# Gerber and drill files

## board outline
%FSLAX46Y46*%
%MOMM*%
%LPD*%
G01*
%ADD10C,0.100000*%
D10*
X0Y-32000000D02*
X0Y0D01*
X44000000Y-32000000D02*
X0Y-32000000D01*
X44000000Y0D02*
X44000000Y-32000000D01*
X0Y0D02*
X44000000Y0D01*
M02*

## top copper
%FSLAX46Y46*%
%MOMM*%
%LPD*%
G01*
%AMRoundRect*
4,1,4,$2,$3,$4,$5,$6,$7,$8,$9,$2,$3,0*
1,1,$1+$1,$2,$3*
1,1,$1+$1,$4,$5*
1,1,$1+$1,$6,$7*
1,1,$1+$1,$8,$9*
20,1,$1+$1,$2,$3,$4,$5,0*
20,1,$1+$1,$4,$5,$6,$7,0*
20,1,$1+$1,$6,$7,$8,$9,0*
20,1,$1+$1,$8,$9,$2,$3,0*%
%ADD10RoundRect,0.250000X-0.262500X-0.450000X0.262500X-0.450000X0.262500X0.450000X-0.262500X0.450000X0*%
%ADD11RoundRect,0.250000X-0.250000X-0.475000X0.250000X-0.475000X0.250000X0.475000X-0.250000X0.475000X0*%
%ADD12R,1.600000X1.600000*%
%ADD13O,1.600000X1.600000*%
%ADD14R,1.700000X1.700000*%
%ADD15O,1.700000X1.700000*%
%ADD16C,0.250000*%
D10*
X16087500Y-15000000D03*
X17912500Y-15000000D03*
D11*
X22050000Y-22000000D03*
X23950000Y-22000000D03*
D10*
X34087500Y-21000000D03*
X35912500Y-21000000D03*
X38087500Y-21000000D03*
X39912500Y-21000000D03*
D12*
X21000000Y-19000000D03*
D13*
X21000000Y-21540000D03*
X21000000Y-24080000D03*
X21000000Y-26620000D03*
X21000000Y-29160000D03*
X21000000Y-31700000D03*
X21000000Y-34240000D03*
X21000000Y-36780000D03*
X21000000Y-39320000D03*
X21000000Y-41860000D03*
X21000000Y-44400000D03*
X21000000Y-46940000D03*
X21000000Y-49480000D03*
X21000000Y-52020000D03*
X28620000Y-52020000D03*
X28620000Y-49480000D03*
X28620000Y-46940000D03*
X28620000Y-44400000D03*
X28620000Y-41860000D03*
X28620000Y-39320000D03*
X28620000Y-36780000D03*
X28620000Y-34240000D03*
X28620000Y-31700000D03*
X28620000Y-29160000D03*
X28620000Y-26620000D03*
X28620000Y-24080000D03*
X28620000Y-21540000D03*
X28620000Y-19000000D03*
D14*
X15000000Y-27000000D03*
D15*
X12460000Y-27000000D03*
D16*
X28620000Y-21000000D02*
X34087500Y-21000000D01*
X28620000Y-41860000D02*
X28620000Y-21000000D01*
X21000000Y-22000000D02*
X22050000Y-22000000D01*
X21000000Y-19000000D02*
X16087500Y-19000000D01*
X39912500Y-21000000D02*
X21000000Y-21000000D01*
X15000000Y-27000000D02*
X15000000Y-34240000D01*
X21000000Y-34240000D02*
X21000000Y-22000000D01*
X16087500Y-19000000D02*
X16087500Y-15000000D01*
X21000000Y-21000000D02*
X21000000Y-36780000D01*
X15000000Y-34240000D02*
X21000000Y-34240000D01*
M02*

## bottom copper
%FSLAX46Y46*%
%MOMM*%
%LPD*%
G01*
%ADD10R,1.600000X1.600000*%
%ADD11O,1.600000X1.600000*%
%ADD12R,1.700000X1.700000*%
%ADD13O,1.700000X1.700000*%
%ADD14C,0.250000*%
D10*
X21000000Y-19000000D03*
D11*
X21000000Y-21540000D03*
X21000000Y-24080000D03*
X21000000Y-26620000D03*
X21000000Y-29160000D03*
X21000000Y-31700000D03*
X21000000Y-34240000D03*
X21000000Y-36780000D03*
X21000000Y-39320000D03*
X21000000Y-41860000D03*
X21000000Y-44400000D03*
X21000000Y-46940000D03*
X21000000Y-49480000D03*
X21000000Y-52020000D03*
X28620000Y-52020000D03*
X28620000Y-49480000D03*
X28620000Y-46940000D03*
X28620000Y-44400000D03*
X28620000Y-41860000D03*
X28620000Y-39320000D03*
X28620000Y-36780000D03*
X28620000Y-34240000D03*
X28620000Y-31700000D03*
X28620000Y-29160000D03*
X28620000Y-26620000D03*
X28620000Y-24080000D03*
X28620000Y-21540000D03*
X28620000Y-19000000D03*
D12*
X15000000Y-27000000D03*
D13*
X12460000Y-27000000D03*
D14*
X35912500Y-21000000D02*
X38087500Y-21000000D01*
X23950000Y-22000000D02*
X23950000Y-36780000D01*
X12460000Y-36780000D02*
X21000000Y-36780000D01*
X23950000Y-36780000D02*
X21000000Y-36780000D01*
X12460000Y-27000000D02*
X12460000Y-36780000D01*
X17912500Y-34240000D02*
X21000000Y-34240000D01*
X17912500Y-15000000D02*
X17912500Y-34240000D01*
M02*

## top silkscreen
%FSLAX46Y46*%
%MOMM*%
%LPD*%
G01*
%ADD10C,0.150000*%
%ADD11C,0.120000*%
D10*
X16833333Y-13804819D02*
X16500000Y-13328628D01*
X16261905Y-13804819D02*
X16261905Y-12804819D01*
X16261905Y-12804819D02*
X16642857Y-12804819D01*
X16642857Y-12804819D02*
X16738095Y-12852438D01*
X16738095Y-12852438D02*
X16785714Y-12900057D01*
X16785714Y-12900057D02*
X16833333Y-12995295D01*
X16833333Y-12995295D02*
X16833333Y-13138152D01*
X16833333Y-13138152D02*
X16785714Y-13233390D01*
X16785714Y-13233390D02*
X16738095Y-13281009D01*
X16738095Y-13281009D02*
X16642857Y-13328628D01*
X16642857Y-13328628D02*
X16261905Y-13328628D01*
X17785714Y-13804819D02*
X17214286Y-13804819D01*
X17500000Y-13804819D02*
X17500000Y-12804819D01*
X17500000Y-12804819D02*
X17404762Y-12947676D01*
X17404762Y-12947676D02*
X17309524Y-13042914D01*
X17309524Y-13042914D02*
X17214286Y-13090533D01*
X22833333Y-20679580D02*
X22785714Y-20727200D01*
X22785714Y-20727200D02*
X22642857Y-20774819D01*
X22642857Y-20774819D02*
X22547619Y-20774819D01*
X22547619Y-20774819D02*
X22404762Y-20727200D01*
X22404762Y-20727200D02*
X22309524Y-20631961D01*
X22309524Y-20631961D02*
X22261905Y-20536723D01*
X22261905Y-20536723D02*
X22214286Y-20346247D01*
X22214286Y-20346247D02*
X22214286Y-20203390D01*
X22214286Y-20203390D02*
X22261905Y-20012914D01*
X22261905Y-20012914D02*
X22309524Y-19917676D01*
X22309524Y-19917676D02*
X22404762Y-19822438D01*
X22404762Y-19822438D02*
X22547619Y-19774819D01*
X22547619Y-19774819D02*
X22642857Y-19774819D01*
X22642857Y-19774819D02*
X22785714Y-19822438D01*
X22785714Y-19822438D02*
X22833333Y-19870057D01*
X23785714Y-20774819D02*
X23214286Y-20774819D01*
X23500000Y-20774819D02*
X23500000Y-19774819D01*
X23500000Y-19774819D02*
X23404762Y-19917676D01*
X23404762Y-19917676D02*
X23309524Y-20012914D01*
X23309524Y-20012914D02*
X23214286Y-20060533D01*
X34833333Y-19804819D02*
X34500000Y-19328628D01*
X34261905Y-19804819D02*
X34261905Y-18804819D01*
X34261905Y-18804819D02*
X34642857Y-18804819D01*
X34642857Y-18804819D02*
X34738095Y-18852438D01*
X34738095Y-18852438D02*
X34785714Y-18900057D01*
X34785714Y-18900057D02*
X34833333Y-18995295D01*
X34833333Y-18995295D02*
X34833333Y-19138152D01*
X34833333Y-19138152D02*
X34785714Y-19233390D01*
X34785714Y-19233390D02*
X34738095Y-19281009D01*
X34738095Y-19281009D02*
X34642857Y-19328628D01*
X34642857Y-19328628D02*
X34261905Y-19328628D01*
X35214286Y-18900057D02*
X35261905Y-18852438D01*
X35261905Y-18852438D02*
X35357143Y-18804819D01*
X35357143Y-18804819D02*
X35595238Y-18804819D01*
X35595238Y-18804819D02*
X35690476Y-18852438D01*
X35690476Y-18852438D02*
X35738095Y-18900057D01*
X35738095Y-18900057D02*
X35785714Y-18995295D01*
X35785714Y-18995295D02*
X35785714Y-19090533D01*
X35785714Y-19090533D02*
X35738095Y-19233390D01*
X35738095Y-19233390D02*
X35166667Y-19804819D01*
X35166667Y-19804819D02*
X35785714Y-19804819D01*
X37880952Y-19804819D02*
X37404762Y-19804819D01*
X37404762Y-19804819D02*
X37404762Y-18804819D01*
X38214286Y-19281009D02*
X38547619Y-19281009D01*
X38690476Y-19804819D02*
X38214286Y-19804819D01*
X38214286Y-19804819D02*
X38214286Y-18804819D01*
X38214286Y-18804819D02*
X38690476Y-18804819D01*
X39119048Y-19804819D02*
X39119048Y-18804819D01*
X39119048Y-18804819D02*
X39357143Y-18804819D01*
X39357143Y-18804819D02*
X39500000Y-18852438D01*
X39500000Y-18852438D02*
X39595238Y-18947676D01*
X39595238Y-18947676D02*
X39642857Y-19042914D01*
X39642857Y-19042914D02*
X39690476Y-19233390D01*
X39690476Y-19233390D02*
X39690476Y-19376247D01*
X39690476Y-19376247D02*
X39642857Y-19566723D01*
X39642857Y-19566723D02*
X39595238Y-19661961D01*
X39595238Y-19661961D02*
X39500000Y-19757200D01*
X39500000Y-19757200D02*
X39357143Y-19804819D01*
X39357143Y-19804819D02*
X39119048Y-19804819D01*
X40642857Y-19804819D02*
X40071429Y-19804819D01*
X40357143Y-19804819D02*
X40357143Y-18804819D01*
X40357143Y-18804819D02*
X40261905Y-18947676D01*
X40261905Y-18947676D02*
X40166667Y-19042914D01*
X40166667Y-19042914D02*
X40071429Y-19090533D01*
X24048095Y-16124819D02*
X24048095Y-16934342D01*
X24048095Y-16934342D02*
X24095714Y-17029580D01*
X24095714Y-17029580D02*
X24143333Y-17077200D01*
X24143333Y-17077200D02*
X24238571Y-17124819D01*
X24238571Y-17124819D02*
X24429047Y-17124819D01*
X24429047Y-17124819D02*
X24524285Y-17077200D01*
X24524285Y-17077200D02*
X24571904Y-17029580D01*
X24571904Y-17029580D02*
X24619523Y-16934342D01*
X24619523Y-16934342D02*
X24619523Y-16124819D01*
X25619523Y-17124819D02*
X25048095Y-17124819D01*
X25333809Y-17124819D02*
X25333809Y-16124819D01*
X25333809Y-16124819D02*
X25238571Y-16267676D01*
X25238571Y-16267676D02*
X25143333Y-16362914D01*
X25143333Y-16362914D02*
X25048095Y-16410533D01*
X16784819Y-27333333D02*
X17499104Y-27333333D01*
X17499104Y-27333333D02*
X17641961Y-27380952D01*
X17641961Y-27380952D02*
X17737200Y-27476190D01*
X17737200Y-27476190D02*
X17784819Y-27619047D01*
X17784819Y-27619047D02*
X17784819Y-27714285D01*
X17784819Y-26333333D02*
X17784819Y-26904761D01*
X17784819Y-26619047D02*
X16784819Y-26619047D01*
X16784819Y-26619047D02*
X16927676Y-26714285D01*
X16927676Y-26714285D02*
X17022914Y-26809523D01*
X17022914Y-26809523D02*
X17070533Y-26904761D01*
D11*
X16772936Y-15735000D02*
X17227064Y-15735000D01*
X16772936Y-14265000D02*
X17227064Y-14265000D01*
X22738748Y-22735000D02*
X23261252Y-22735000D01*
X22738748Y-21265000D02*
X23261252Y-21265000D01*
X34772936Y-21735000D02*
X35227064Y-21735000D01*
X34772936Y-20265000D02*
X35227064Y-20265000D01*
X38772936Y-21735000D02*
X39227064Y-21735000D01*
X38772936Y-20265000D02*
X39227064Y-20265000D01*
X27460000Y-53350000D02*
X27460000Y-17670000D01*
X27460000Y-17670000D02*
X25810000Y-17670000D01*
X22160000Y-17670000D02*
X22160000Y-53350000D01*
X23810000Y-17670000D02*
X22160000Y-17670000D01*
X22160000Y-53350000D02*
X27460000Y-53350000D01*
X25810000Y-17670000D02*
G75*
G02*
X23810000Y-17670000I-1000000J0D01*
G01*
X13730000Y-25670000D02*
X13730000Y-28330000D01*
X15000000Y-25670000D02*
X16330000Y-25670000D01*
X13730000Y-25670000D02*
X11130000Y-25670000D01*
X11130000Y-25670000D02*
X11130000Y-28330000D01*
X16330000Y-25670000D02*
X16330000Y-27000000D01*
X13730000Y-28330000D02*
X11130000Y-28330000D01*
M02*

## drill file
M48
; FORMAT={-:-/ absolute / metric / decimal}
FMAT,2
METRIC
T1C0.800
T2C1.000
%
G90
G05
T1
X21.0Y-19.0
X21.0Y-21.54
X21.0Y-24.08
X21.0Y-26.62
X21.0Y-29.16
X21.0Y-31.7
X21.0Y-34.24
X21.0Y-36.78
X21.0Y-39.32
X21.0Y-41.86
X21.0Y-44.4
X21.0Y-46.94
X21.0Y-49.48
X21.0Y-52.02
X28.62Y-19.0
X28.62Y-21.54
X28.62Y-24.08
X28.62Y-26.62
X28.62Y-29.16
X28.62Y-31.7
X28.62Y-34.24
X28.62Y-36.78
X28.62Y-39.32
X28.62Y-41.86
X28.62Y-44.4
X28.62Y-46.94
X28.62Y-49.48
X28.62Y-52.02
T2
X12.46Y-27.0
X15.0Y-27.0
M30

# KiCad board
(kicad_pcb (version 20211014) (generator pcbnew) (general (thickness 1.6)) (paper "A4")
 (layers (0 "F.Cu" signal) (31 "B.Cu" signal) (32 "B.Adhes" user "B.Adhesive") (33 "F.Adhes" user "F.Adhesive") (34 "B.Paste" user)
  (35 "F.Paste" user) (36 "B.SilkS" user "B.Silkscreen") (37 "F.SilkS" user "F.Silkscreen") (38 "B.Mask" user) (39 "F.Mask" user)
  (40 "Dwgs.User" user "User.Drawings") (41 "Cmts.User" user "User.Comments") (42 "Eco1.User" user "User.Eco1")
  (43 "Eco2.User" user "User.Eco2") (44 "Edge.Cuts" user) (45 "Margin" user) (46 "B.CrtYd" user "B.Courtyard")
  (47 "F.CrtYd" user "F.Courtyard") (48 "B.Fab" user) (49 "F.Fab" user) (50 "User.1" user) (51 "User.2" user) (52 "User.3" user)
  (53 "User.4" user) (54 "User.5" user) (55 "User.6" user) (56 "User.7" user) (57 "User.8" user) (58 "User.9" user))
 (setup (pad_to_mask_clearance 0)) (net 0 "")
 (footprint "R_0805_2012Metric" (layer "F.Cu") (at 17 15)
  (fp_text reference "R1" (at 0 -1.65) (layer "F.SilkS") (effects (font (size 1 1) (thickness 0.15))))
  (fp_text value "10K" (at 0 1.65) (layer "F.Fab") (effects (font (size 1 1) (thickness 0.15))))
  (fp_line (start -0.227064 0.735) (end 0.227064 0.735) (layer "F.SilkS") (width 0.12))
  (fp_line (start -0.227064 -0.735) (end 0.227064 -0.735) (layer "F.SilkS") (width 0.12))
  (pad "1" smd roundrect (at -0.9125 0) (size 1.025 1.4) (layers "F.Cu" "F.Paste" "F.Mask") (roundrect_rratio 0.243902))
  (pad "2" smd roundrect (at 0.9125 0) (size 1.025 1.4) (layers "F.Cu" "F.Paste" "F.Mask") (roundrect_rratio 0.243902)))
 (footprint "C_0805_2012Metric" (layer "F.Cu") (at 23 22)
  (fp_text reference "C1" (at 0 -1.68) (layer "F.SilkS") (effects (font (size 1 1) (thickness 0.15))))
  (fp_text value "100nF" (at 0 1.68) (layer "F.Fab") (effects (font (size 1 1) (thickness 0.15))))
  (fp_line (start -0.261252 0.735) (end 0.261252 0.735) (layer "F.SilkS") (width 0.12))
  (fp_line (start -0.261252 -0.735) (end 0.261252 -0.735) (layer "F.SilkS") (width 0.12))
  (pad "1" smd roundrect (at -0.95 0) (size 1 1.45) (layers "F.Cu" "F.Paste" "F.Mask") (roundrect_rratio 0.25))
  (pad "2" smd roundrect (at 0.95 0) (size 1 1.45) (layers "F.Cu" "F.Paste" "F.Mask") (roundrect_rratio 0.25)))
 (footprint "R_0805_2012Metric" (layer "F.Cu") (at 35 21)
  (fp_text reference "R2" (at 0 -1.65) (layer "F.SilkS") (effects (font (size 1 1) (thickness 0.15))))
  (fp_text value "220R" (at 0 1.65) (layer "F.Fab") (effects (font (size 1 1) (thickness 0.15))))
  (fp_line (start -0.227064 0.735) (end 0.227064 0.735) (layer "F.SilkS") (width 0.12))
  (fp_line (start -0.227064 -0.735) (end 0.227064 -0.735) (layer "F.SilkS") (width 0.12))
  (pad "1" smd roundrect (at -0.9125 0) (size 1.025 1.4) (layers "F.Cu" "F.Paste" "F.Mask") (roundrect_rratio 0.243902))
  (pad "2" smd roundrect (at 0.9125 0) (size 1.025 1.4) (layers "F.Cu" "F.Paste" "F.Mask") (roundrect_rratio 0.243902)))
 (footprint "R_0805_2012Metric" (layer "F.Cu") (at 39 21)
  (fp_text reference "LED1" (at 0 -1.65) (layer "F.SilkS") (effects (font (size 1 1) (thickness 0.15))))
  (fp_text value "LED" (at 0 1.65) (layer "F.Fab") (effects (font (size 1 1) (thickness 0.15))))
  (fp_line (start -0.227064 0.735) (end 0.227064 0.735) (layer "F.SilkS") (width 0.12))
  (fp_line (start -0.227064 -0.735) (end 0.227064 -0.735) (layer "F.SilkS") (width 0.12))
  (pad "1" smd roundrect (at -0.9125 0) (size 1.025 1.4) (layers "F.Cu" "F.Paste" "F.Mask") (roundrect_rratio 0.243902))
  (pad "2" smd roundrect (at 0.9125 0) (size 1.025 1.4) (layers "F.Cu" "F.Paste" "F.Mask") (roundrect_rratio 0.243902)))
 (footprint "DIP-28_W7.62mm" (layer "F.Cu") (at 21 19)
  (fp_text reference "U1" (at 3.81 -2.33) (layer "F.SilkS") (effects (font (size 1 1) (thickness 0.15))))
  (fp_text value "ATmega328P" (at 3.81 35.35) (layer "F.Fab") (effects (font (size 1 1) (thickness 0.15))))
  (fp_line (start 6.46 34.35) (end 6.46 -1.33) (layer "F.SilkS") (width 0.12))
  (fp_line (start 6.46 -1.33) (end 4.81 -1.33) (layer "F.SilkS") (width 0.12))
  (fp_line (start 1.16 -1.33) (end 1.16 34.35) (layer "F.SilkS") (width 0.12))
  (fp_line (start 2.81 -1.33) (end 1.16 -1.33) (layer "F.SilkS") (width 0.12))
  (fp_line (start 1.16 34.35) (end 6.46 34.35) (layer "F.SilkS") (width 0.12))
  (fp_arc (start 4.81 -1.33) (mid 3.81 -0.33) (end 2.81 -1.33) (layer "F.SilkS") (width 0.12))
  (pad "1" thru_hole rect (at 0 0) (size 1.6 1.6) (drill 0.8) (layers *.Cu *.Mask))
  (pad "2" thru_hole oval (at 0 2.54) (size 1.6 1.6) (drill 0.8) (layers *.Cu *.Mask))
  (pad "3" thru_hole oval (at 0 5.08) (size 1.6 1.6) (drill 0.8) (layers *.Cu *.Mask))
  (pad "4" thru_hole oval (at 0 7.62) (size 1.6 1.6) (drill 0.8) (layers *.Cu *.Mask))
  (pad "5" thru_hole oval (at 0 10.16) (size 1.6 1.6) (drill 0.8) (layers *.Cu *.Mask))
  (pad "6" thru_hole oval (at 0 12.7) (size 1.6 1.6) (drill 0.8) (layers *.Cu *.Mask))
  (pad "7" thru_hole oval (at 0 15.24) (size 1.6 1.6) (drill 0.8) (layers *.Cu *.Mask))
  (pad "8" thru_hole oval (at 0 17.78) (size 1.6 1.6) (drill 0.8) (layers *.Cu *.Mask))
  (pad "9" thru_hole oval (at 0 20.32) (size 1.6 1.6) (drill 0.8) (layers *.Cu *.Mask))
  (pad "10" thru_hole oval (at 0 22.86) (size 1.6 1.6) (drill 0.8) (layers *.Cu *.Mask))
  (pad "11" thru_hole oval (at 0 25.4) (size 1.6 1.6) (drill 0.8) (layers *.Cu *.Mask))
  (pad "12" thru_hole oval (at 0 27.94) (size 1.6 1.6) (drill 0.8) (layers *.Cu *.Mask))
  (pad "13" thru_hole oval (at 0 30.48) (size 1.6 1.6) (drill 0.8) (layers *.Cu *.Mask))
  (pad "14" thru_hole oval (at 0 33.02) (size 1.6 1.6) (drill 0.8) (layers *.Cu *.Mask))
  (pad "15" thru_hole oval (at 7.62 33.02) (size 1.6 1.6) (drill 0.8) (layers *.Cu *.Mask))
  (pad "16" thru_hole oval (at 7.62 30.48) (size 1.6 1.6) (drill 0.8) (layers *.Cu *.Mask))
  (pad "17" thru_hole oval (at 7.62 27.94) (size 1.6 1.6) (drill 0.8) (layers *.Cu *.Mask))
  (pad "18" thru_hole oval (at 7.62 25.4) (size 1.6 1.6) (drill 0.8) (layers *.Cu *.Mask))
  (pad "19" thru_hole oval (at 7.62 22.86) (size 1.6 1.6) (drill 0.8) (layers *.Cu *.Mask))
  (pad "20" thru_hole oval (at 7.62 20.32) (size 1.6 1.6) (drill 0.8) (layers *.Cu *.Mask))
  (pad "21" thru_hole oval (at 7.62 17.78) (size 1.6 1.6) (drill 0.8) (layers *.Cu *.Mask))
  (pad "22" thru_hole oval (at 7.62 15.24) (size 1.6 1.6) (drill 0.8) (layers *.Cu *.Mask))
  (pad "23" thru_hole oval (at 7.62 12.7) (size 1.6 1.6) (drill 0.8) (layers *.Cu *.Mask))
  (pad "24" thru_hole oval (at 7.62 10.16) (size 1.6 1.6) (drill 0.8) (layers *.Cu *.Mask))
  (pad "25" thru_hole oval (at 7.62 7.62) (size 1.6 1.6) (drill 0.8) (layers *.Cu *.Mask))
  (pad "26" thru_hole oval (at 7.62 5.08) (size 1.6 1.6) (drill 0.8) (layers *.Cu *.Mask))
  (pad "27" thru_hole oval (at 7.62 2.54) (size 1.6 1.6) (drill 0.8) (layers *.Cu *.Mask))
  (pad "28" thru_hole oval (at 7.62 0) (size 1.6 1.6) (drill 0.8) (layers *.Cu *.Mask)))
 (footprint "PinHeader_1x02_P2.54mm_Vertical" (layer "F.Cu") (at 15 27 -90)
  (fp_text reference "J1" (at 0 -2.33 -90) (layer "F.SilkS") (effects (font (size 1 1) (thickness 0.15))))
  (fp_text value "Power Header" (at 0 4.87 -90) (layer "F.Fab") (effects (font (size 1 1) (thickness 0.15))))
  (fp_line (start -1.33 1.27) (end 1.33 1.27) (layer "F.SilkS") (width 0.12))
  (fp_line (start -1.33 0) (end -1.33 -1.33) (layer "F.SilkS") (width 0.12))
  (fp_line (start -1.33 1.27) (end -1.33 3.87) (layer "F.SilkS") (width 0.12))
  (fp_line (start -1.33 3.87) (end 1.33 3.87) (layer "F.SilkS") (width 0.12))
  (fp_line (start -1.33 -1.33) (end 0 -1.33) (layer "F.SilkS") (width 0.12))
  (fp_line (start 1.33 1.27) (end 1.33 3.87) (layer "F.SilkS") (width 0.12))
  (pad "1" thru_hole rect (at 0 0 270) (size 1.7 1.7) (drill 1) (layers *.Cu *.Mask))
  (pad "2" thru_hole oval (at 0 2.54 270) (size 1.7 1.7) (drill 1) (layers *.Cu *.Mask)))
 (gr_line (start 0 32) (end 0 0) (layer "Edge.Cuts") (width 0.1))
 (gr_line (start 44 32) (end 0 32) (layer "Edge.Cuts") (width 0.1))
 (gr_line (start 44 0) (end 44 32) (layer "Edge.Cuts") (width 0.1))
 (gr_line (start 0 0) (end 44 0) (layer "Edge.Cuts") (width 0.1))
 (segment (start 28.62 21) (end 34.0875 21) (width 0.25) (layer "F.Cu") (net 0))
 (segment (start 28.62 41.86) (end 28.62 21) (width 0.25) (layer "F.Cu") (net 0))
 (segment (start 21 22) (end 22.05 22) (width 0.25) (layer "F.Cu") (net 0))
 (segment (start 21 19) (end 16.0875 19) (width 0.25) (layer "F.Cu") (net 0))
 (segment (start 39.9125 21) (end 21 21) (width 0.25) (layer "F.Cu") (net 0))
 (segment (start 15 27) (end 15 34.24) (width 0.25) (layer "F.Cu") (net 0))
 (segment (start 21 34.24) (end 21 22) (width 0.25) (layer "F.Cu") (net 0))
 (segment (start 16.0875 19) (end 16.0875 15) (width 0.25) (layer "F.Cu") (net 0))
 (segment (start 21 21) (end 21 36.78) (width 0.25) (layer "F.Cu") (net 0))
 (segment (start 15 34.24) (end 21 34.24) (width 0.25) (layer "F.Cu") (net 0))
 (segment (start 35.9125 21) (end 38.0875 21) (width 0.25) (layer "B.Cu") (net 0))
 (segment (start 23.95 22) (end 23.95 36.78) (width 0.25) (layer "B.Cu") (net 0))
 (segment (start 12.46 36.78) (end 21 36.78) (width 0.25) (layer "B.Cu") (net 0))
 (segment (start 23.95 36.78) (end 21 36.78) (width 0.25) (layer "B.Cu") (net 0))
 (segment (start 12.46 27) (end 12.46 36.78) (width 0.25) (layer "B.Cu") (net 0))
 (segment (start 17.9125 34.24) (end 21 34.24) (width 0.25) (layer "B.Cu") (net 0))
 (segment (start 17.9125 15) (end 17.9125 34.24) (width 0.25) (layer "B.Cu") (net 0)))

